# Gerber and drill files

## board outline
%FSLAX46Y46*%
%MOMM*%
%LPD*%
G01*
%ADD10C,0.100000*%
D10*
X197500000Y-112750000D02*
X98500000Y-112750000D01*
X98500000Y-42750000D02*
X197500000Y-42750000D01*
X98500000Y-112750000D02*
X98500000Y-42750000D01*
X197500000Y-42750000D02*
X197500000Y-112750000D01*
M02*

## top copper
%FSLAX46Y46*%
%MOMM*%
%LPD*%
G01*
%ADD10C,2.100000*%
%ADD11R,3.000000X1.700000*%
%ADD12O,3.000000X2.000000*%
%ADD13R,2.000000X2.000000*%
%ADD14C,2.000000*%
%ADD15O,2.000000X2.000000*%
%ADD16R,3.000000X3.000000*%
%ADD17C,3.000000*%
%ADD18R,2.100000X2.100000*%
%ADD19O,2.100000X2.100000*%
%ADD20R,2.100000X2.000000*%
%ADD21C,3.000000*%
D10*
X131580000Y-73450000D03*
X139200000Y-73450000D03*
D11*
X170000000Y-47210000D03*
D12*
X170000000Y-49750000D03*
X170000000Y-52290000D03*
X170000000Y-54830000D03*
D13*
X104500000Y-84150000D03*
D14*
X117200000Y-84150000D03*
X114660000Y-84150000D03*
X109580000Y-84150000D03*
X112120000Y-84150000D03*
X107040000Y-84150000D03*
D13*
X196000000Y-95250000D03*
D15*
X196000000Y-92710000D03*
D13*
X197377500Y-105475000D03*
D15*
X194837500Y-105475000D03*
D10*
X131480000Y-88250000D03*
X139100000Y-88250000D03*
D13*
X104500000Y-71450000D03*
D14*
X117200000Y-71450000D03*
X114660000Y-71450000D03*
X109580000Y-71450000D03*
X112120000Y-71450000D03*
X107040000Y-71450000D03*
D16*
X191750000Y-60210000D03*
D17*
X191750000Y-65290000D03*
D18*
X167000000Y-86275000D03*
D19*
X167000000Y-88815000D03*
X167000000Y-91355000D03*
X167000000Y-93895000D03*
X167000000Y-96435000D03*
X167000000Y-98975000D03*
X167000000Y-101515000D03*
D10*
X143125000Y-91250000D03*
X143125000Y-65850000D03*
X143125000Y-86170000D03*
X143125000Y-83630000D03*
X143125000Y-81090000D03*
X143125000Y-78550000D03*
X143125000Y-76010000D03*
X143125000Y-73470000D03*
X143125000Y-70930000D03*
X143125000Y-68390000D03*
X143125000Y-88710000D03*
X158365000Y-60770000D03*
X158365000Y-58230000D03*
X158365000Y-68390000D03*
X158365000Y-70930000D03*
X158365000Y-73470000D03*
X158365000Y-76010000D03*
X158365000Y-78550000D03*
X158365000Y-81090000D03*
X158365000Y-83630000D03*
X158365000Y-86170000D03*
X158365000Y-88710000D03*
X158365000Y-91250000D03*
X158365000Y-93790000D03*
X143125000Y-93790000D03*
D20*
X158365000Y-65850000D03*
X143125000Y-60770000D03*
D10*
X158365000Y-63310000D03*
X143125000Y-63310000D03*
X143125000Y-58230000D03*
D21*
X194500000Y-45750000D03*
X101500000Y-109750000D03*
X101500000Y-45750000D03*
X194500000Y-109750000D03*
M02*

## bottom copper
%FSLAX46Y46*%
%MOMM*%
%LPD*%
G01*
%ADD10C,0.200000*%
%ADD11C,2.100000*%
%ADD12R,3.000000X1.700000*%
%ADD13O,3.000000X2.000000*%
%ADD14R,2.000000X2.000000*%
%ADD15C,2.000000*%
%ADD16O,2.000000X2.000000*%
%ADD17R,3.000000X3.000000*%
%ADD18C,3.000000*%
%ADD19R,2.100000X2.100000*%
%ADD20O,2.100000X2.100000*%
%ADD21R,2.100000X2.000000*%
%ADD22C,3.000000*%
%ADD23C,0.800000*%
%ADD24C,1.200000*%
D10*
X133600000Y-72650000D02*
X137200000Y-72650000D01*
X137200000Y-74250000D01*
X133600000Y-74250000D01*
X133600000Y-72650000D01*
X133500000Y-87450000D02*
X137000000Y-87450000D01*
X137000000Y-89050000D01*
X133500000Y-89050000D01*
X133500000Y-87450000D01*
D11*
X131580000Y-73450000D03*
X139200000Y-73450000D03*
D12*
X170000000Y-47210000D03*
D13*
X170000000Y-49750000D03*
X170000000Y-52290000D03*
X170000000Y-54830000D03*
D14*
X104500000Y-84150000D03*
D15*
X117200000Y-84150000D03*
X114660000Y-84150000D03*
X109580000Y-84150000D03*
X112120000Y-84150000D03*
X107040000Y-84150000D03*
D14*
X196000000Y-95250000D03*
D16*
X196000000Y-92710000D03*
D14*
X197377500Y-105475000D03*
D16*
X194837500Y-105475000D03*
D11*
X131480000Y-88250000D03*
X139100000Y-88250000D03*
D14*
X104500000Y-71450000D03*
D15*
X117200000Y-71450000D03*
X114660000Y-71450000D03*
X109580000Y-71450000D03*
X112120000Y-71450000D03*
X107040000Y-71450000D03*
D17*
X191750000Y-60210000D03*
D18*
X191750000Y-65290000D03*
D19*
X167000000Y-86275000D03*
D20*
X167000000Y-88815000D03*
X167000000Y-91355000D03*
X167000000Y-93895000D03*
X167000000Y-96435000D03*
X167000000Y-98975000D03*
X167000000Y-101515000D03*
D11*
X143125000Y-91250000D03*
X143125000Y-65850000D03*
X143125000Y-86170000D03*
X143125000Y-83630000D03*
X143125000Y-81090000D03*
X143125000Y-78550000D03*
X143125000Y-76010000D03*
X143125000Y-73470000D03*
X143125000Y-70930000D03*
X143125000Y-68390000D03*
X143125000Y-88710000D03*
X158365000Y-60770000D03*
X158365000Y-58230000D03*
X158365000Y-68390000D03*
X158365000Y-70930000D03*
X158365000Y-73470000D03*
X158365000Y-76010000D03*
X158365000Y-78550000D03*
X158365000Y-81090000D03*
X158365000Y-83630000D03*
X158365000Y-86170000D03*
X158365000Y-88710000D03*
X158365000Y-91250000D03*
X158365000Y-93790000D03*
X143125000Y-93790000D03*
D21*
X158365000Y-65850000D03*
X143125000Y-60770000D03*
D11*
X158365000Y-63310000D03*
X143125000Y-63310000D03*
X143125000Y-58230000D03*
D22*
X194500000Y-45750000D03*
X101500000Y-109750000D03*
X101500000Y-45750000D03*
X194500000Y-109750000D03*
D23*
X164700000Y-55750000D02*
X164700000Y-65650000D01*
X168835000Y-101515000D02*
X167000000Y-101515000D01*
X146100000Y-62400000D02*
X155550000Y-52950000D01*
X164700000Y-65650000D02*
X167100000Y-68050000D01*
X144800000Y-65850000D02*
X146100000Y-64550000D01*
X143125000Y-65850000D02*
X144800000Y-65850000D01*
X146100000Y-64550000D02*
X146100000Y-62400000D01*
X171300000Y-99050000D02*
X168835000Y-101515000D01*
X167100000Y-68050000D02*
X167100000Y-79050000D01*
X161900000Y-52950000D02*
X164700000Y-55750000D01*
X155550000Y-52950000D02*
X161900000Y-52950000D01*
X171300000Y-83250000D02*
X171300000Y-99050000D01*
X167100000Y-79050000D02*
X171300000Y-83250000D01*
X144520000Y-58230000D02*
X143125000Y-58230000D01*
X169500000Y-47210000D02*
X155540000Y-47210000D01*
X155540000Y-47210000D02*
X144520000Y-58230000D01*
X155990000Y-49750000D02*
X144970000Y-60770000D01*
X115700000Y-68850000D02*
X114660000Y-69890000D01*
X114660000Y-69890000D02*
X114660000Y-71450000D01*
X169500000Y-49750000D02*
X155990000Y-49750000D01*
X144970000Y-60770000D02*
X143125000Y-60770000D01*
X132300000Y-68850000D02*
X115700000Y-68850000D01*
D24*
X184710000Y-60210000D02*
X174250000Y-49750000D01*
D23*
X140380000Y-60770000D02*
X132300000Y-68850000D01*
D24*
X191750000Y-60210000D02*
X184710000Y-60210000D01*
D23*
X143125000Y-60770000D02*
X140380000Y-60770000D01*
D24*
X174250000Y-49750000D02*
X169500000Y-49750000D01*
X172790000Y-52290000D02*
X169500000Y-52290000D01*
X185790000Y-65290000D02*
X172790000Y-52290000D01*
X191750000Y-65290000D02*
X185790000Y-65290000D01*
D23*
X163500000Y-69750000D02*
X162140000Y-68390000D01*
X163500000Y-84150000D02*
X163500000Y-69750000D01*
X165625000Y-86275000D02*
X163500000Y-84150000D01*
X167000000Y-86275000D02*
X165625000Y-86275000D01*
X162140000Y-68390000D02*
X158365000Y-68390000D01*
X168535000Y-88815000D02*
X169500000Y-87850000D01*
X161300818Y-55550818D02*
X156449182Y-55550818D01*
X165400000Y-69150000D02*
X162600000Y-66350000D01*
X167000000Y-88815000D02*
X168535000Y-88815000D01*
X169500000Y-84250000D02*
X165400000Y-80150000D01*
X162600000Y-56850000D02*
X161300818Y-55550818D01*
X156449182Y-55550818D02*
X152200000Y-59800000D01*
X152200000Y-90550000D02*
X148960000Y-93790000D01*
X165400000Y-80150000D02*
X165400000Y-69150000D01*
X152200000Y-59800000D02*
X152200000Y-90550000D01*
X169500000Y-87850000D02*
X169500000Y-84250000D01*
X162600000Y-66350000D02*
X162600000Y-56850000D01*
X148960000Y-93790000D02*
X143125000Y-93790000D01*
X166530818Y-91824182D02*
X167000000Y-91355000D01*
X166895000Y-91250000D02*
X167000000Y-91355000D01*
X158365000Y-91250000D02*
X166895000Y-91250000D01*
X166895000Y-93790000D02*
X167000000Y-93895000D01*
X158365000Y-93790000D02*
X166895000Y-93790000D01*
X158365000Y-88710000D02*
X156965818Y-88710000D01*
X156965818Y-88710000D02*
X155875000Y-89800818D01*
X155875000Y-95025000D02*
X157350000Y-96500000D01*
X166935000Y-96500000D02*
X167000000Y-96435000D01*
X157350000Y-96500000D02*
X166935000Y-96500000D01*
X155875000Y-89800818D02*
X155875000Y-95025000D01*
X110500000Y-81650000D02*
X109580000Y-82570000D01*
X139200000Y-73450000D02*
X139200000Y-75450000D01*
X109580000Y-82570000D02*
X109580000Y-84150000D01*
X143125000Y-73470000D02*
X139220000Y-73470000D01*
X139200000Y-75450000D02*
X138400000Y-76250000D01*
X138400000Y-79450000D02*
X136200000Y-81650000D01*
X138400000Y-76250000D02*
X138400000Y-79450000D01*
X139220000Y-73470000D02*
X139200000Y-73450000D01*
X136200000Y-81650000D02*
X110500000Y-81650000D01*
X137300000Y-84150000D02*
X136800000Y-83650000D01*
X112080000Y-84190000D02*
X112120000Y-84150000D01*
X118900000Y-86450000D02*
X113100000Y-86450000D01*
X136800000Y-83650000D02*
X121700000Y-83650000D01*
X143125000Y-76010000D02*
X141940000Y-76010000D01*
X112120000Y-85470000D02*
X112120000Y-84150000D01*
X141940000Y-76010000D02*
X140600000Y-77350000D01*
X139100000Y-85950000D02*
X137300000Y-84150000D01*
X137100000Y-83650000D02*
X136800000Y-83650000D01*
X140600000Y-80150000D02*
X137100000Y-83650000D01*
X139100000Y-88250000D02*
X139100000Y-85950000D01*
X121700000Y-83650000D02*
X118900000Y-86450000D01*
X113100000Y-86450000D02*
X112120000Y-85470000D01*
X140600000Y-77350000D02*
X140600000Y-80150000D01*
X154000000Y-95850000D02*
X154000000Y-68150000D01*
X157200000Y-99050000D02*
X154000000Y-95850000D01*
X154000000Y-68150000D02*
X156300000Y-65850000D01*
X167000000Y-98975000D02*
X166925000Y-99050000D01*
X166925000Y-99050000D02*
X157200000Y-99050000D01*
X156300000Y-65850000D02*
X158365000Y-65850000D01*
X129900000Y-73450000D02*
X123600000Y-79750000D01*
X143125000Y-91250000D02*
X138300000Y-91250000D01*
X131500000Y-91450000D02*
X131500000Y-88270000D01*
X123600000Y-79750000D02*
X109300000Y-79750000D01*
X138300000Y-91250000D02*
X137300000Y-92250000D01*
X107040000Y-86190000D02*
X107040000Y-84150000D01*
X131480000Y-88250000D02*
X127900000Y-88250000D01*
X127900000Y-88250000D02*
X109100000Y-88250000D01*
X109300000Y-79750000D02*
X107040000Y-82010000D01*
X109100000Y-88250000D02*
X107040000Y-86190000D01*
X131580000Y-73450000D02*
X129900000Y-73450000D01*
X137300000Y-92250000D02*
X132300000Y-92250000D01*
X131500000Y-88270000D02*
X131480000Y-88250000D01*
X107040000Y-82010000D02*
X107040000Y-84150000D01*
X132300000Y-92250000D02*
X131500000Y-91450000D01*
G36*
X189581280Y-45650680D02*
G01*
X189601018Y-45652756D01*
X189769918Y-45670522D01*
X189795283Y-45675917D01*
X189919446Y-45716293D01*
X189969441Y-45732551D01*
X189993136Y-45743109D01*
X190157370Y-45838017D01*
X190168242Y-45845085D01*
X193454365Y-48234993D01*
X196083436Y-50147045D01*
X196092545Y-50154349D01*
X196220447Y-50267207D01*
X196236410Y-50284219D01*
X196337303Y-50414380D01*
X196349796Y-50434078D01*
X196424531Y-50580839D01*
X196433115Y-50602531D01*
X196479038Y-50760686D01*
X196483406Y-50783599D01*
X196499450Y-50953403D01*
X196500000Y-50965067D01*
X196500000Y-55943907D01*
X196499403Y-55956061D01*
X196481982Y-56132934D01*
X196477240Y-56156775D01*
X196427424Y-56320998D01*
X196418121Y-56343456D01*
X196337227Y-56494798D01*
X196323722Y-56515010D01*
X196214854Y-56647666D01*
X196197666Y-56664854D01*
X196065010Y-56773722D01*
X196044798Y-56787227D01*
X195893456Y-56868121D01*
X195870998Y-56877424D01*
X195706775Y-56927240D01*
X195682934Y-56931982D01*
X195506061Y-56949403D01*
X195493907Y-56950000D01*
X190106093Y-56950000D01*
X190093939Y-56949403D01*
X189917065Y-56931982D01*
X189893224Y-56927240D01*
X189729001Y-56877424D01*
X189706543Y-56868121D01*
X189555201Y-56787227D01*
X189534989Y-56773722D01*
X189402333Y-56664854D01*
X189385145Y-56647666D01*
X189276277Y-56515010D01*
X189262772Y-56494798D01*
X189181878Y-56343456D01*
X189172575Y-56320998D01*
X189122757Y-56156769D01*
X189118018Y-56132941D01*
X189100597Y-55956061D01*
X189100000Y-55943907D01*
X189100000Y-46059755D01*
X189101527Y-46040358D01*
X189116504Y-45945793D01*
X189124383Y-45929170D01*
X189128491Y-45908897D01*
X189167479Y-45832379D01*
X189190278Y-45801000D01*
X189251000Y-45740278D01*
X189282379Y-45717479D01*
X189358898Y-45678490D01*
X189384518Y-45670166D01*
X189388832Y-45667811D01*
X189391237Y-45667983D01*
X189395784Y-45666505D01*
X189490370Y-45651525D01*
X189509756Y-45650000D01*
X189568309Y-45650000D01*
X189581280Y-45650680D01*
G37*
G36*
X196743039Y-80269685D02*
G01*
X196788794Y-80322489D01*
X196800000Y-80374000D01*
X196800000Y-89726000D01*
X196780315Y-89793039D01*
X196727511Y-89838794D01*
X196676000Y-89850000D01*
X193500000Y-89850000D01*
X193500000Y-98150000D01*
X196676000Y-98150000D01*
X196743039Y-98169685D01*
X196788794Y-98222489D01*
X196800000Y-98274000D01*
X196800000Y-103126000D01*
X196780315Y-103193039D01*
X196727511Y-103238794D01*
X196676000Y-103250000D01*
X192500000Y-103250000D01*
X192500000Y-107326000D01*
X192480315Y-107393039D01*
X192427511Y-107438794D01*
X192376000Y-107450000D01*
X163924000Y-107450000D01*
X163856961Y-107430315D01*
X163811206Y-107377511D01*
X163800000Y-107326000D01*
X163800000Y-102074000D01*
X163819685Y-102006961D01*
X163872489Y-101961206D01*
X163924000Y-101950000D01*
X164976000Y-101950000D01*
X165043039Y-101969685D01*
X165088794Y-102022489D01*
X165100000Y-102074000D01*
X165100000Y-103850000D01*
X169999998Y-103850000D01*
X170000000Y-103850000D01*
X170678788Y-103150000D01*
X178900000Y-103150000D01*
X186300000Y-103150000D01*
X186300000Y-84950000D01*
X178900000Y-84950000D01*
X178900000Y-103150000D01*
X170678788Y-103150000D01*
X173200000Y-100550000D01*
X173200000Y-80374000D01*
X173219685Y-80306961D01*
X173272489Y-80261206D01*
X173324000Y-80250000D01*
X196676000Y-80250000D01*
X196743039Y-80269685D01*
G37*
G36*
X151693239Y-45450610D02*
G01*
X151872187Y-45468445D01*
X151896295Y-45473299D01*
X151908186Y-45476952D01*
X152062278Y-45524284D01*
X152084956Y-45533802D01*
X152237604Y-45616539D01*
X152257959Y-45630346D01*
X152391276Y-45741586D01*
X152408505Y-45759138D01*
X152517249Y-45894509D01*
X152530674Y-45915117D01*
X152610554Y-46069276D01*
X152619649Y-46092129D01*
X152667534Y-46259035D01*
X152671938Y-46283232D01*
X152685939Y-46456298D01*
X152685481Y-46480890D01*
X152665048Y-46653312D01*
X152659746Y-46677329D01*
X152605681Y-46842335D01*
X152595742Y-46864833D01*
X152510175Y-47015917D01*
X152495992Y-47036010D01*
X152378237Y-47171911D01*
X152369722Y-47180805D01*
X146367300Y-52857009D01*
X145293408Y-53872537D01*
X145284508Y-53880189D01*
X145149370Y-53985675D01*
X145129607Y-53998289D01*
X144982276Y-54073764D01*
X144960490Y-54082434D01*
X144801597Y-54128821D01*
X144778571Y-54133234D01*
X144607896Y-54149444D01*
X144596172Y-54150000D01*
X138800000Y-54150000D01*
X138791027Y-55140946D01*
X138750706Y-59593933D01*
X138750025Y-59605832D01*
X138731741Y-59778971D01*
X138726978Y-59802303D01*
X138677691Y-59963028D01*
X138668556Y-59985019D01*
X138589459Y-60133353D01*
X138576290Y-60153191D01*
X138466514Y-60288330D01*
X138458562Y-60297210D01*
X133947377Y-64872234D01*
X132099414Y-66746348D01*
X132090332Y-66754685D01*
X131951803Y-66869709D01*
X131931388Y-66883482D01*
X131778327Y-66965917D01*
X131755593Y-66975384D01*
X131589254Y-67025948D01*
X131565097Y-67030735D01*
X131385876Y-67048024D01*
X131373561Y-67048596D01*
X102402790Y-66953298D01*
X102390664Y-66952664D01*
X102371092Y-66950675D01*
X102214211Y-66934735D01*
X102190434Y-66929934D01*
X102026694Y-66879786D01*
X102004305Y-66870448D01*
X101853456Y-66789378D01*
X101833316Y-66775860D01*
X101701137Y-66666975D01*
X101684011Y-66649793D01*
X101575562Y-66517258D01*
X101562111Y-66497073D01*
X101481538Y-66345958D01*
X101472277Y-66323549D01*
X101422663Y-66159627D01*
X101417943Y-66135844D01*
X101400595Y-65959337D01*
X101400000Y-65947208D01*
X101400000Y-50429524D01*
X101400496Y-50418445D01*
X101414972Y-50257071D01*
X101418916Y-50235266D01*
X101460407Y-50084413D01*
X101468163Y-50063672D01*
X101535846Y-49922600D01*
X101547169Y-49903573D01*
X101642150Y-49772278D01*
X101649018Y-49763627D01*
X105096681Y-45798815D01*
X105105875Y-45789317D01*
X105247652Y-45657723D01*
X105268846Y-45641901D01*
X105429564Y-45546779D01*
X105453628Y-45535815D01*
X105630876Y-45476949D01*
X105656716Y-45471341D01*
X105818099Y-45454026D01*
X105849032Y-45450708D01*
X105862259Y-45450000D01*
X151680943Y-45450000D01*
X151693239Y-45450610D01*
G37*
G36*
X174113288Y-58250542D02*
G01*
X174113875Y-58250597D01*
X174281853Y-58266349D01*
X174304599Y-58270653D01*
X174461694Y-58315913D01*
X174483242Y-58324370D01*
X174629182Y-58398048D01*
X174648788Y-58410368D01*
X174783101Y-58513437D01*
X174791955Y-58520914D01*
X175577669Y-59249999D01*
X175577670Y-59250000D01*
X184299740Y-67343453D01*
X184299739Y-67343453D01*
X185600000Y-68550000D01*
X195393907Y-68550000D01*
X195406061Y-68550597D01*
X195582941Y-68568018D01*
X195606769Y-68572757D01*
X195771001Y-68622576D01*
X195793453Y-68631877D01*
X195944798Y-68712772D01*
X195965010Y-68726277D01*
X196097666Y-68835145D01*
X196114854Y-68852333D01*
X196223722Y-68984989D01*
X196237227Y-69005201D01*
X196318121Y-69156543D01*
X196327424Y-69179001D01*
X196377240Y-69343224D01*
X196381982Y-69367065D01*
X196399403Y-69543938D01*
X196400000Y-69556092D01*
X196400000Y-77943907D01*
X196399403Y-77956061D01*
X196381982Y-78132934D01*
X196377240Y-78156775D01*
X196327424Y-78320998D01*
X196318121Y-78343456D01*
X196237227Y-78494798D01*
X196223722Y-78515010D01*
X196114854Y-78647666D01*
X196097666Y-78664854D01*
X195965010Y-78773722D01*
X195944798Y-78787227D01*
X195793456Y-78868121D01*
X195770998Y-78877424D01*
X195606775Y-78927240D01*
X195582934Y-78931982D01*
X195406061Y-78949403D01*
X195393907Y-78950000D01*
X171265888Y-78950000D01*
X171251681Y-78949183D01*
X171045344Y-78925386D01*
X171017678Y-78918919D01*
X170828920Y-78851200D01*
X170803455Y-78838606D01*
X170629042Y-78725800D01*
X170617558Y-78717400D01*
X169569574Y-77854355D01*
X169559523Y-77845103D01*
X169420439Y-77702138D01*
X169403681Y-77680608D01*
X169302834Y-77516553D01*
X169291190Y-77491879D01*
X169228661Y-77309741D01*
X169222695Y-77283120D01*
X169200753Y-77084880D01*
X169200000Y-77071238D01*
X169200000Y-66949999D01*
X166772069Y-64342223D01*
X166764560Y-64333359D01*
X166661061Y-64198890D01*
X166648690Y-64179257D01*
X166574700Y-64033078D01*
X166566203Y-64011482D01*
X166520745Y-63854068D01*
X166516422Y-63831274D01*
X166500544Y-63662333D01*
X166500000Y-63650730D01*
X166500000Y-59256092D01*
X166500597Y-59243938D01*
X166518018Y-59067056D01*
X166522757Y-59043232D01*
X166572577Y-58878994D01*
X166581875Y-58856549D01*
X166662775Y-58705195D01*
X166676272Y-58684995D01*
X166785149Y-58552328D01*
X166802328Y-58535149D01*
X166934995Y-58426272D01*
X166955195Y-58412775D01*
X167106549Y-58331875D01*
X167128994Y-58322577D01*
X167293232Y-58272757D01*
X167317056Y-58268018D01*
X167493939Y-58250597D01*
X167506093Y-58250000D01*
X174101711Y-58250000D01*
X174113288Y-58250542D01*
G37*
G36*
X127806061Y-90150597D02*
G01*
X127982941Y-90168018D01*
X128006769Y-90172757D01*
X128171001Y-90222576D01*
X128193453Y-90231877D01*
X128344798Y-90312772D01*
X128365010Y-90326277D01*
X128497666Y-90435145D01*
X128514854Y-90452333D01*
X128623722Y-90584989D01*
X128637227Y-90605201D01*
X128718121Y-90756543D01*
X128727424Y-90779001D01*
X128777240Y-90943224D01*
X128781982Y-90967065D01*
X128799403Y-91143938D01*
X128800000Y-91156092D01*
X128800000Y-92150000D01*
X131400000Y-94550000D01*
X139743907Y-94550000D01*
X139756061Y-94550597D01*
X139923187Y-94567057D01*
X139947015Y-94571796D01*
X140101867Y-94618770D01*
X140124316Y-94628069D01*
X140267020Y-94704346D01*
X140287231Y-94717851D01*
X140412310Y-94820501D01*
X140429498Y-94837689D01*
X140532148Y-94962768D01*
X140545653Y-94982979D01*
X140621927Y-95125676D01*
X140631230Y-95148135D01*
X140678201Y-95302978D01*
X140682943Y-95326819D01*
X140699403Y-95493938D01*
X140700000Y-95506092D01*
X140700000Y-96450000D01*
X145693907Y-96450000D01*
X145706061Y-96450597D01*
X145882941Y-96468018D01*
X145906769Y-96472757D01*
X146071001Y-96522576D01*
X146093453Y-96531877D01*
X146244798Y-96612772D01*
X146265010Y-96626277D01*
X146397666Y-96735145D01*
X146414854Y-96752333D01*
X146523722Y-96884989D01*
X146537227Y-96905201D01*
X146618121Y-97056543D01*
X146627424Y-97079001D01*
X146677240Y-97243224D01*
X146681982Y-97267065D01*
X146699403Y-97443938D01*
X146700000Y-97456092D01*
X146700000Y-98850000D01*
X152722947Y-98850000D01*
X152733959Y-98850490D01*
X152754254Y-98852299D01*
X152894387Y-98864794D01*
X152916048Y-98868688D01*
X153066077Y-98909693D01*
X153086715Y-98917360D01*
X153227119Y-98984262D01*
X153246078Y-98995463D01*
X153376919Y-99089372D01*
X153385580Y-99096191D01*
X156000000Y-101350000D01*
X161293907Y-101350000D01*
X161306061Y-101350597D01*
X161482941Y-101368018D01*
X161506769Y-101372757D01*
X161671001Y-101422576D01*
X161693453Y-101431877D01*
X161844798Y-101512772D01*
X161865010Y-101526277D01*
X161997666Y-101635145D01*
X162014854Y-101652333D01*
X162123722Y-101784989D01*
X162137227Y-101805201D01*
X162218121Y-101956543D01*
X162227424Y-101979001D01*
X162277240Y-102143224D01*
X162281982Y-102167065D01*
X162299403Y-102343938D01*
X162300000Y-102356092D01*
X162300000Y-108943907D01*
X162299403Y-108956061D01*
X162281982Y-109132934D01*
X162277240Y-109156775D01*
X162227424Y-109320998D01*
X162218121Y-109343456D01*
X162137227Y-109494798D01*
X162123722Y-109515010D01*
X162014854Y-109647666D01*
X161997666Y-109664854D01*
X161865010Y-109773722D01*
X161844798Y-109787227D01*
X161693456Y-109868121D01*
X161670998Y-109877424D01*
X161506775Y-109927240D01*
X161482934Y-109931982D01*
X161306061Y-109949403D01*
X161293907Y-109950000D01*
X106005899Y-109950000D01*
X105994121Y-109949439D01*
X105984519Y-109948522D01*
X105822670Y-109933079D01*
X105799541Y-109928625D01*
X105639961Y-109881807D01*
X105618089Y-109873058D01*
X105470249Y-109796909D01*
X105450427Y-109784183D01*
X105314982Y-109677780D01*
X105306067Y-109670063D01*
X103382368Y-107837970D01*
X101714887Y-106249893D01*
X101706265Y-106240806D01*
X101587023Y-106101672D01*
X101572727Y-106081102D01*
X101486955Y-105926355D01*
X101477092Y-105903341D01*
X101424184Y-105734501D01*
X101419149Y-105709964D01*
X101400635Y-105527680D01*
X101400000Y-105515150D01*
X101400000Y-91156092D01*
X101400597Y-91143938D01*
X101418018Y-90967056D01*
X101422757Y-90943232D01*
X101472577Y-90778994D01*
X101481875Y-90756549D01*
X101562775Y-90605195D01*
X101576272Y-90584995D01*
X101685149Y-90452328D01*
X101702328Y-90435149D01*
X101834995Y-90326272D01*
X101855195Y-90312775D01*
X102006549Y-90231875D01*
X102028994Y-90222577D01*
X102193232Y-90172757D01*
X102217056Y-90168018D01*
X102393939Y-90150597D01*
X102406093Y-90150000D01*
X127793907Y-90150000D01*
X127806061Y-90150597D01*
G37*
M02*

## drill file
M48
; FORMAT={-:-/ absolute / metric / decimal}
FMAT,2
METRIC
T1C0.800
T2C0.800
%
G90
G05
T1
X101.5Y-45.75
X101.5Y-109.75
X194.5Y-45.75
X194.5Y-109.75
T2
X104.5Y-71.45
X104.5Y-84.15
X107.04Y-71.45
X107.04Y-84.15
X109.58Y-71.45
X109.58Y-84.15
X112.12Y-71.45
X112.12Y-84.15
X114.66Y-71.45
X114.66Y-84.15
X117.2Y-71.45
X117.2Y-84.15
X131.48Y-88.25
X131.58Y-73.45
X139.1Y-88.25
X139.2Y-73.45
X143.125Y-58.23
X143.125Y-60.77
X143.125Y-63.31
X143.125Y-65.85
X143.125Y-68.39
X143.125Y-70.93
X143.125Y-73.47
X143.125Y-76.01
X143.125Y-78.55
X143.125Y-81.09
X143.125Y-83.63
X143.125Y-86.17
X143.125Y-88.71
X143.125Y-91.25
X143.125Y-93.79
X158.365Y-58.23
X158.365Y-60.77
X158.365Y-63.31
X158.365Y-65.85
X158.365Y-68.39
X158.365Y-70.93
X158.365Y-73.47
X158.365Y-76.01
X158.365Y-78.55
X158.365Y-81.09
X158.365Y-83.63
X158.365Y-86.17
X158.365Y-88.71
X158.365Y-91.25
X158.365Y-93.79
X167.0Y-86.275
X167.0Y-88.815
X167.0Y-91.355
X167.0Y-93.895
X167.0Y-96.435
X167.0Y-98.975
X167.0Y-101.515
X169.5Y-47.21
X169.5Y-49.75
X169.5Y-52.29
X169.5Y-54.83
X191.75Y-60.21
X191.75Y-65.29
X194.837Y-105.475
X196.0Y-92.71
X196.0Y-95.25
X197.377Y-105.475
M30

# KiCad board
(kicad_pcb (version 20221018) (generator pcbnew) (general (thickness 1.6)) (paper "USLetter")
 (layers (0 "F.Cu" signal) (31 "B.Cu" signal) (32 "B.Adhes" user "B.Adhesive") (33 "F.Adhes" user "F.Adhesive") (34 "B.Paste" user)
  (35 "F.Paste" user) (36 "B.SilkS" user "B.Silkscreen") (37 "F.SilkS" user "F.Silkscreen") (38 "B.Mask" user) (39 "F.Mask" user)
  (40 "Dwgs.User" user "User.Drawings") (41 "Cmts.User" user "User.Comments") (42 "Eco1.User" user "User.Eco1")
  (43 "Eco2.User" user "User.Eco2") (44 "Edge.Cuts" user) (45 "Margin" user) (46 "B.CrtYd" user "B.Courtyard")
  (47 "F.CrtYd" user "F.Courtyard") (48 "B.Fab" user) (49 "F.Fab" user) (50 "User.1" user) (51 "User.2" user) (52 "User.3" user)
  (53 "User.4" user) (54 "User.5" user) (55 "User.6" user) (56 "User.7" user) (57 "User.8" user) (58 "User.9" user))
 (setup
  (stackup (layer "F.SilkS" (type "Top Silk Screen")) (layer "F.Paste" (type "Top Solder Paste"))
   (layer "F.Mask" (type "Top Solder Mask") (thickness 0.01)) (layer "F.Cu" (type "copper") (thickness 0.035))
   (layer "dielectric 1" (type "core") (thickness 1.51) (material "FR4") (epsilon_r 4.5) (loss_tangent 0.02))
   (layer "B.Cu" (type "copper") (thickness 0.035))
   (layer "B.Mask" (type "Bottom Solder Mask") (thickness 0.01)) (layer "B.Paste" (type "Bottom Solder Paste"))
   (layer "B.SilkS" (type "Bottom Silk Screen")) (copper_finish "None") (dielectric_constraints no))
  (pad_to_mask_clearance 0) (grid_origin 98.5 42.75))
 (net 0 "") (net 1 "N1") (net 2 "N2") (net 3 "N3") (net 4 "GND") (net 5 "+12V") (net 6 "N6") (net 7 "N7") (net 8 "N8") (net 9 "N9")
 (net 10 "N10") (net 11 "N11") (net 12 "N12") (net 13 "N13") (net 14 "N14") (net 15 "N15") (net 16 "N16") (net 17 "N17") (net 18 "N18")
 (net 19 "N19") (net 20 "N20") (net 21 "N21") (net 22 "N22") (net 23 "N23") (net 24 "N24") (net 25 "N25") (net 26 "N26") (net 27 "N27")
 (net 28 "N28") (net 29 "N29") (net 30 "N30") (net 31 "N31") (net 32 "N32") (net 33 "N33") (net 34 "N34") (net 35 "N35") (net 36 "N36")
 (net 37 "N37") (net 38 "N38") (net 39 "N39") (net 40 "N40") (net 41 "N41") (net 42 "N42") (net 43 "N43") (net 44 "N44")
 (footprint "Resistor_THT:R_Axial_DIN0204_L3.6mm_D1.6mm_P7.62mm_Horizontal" (layer "F.Cu") (at 131.58 73.45)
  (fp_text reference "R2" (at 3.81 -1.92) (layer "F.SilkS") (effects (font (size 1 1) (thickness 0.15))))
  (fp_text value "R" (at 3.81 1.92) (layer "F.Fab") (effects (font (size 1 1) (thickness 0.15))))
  (pad "1" thru_hole circle (at 0 0) (size 2.1 2.1) (drill 0.8) (layers "*.Cu" "*.Mask") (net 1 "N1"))
  (pad "2" thru_hole circle (at 7.62 0) (size 2.1 2.1) (drill 0.8) (layers "*.Cu" "*.Mask") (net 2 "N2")))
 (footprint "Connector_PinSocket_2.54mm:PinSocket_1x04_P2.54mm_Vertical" (layer "F.Cu") (at 169.5 47.21)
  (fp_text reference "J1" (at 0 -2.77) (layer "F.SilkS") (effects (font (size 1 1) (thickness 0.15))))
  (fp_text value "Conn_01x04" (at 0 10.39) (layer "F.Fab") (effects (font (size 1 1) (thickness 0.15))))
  (pad "1" thru_hole rect (at 0 0) (size 3 1.7) (drill 0.8 (offset 0.5 0)) (layers "*.Cu" "*.Mask") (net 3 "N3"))
  (pad "2" thru_hole oval (at 0 2.54) (size 3 2) (drill 0.8 (offset 0.5 0)) (layers "*.Cu" "*.Mask") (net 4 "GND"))
  (pad "3" thru_hole oval (at 0 5.08) (size 3 2) (drill 0.8 (offset 0.5 0)) (layers "*.Cu" "*.Mask") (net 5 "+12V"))
  (pad "4" thru_hole oval (at 0 7.62) (size 3 2) (drill 0.8 (offset 0.5 0)) (layers "*.Cu" "*.Mask") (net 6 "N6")))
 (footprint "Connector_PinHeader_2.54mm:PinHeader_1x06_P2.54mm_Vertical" (layer "F.Cu") (at 104.5 84.15 90)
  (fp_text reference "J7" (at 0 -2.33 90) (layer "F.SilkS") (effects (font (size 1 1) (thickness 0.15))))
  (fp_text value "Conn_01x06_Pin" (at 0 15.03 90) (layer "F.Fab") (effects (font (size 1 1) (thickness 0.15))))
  (pad "D2" thru_hole rect (at 0 0 90) (size 2 2) (drill 0.8) (layers "*.Cu" "*.Mask") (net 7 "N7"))
  (pad "D3" thru_hole circle (at 0 12.7 90) (size 2 2) (drill 0.8) (layers "*.Cu" "*.Mask") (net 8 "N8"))
  (pad "GND" thru_hole circle (at 0 10.16 90) (size 2 2) (drill 0.8) (layers "*.Cu" "*.Mask") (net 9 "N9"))
  (pad "SCL" thru_hole circle (at 0 5.08 90) (size 2 2) (drill 0.8) (layers "*.Cu" "*.Mask") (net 2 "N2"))
  (pad "SDA" thru_hole circle (at 0 7.62 90) (size 2 2) (drill 0.8) (layers "*.Cu" "*.Mask") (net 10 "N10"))
  (pad "VCC" thru_hole circle (at 0 2.54 90) (size 2 2) (drill 0.8) (layers "*.Cu" "*.Mask") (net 1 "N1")))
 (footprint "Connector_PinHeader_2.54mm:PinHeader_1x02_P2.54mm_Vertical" (layer "F.Cu") (at 196 95.25 180)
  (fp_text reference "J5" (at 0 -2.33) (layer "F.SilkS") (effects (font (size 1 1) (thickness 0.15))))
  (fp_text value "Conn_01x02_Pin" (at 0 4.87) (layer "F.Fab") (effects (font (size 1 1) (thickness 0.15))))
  (pad "1" thru_hole rect (at 0 0 180) (size 2 2) (drill 0.8) (layers "*.Cu" "*.Mask") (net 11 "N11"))
  (pad "2" thru_hole oval (at 0 2.54 180) (size 2 2) (drill 0.8) (layers "*.Cu" "*.Mask") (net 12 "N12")))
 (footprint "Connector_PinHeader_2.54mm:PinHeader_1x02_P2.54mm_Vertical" (layer "F.Cu") (at 197.3775 105.475 -90)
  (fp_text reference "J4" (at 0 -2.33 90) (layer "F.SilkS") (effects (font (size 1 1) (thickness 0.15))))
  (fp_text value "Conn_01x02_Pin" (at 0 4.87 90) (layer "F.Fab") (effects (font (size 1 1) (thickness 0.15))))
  (pad "1" thru_hole rect (at 0 0 270) (size 2 2) (drill 0.8) (layers "*.Cu" "*.Mask") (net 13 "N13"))
  (pad "2" thru_hole oval (at 0 2.54 270) (size 2 2) (drill 0.8) (layers "*.Cu" "*.Mask") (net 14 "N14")))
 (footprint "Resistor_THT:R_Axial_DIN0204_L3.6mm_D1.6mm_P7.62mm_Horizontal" (layer "F.Cu") (at 131.48 88.25)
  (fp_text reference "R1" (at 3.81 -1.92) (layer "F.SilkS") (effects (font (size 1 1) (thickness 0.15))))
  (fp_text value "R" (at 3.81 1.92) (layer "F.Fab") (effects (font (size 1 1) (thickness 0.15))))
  (pad "1" thru_hole circle (at 0 0) (size 2.1 2.1) (drill 0.8) (layers "*.Cu" "*.Mask") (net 1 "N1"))
  (pad "2" thru_hole circle (at 7.62 0) (size 2.1 2.1) (drill 0.8) (layers "*.Cu" "*.Mask") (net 10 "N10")))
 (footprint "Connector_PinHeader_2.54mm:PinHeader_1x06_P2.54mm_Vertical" (layer "F.Cu") (at 104.5 71.45 90)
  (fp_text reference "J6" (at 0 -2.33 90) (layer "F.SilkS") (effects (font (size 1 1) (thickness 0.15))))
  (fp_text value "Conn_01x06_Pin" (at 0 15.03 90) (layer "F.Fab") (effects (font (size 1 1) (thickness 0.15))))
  (pad "D0" thru_hole rect (at 0 0 90) (size 2 2) (drill 0.8) (layers "*.Cu" "*.Mask") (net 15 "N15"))
  (pad "D1" thru_hole circle (at 0 12.7 90) (size 2 2) (drill 0.8) (layers "*.Cu" "*.Mask") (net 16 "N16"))
  (pad "GND" thru_hole circle (at 0 10.16 90) (size 2 2) (drill 0.8) (layers "*.Cu" "*.Mask") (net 4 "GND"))
  (pad "Rx" thru_hole circle (at 0 5.08 90) (size 2 2) (drill 0.8) (layers "*.Cu" "*.Mask") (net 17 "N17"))
  (pad "Tx" thru_hole circle (at 0 7.62 90) (size 2 2) (drill 0.8) (layers "*.Cu" "*.Mask") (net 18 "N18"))
  (pad "VCC" thru_hole circle (at 0 2.54 90) (size 2 2) (drill 0.8) (layers "*.Cu" "*.Mask") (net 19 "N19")))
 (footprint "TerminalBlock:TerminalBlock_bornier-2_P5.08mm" (layer "F.Cu") (at 191.75 60.21 -90)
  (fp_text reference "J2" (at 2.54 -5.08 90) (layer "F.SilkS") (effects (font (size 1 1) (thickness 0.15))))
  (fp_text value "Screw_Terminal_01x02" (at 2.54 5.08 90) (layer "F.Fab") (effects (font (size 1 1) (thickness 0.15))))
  (pad "1" thru_hole rect (at 0 0 270) (size 3 3) (drill 0.8) (layers "*.Cu" "*.Mask") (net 4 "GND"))
  (pad "2" thru_hole circle (at 5.08 0 270) (size 3 3) (drill 0.8) (layers "*.Cu" "*.Mask") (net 5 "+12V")))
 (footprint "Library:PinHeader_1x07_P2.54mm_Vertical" (layer "F.Cu") (at 167 86.275)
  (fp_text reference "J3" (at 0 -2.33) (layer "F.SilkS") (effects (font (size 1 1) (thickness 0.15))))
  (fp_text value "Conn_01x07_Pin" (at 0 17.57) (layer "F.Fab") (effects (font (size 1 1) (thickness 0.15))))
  (pad "1" thru_hole rect (at 0 0) (size 2.1 2.1) (drill 0.8) (layers "*.Cu" "*.Mask") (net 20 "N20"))
  (pad "2" thru_hole oval (at 0 2.54) (size 2.1 2.1) (drill 0.8) (layers "*.Cu" "*.Mask") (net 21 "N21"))
  (pad "3" thru_hole oval (at 0 5.08) (size 2.1 2.1) (drill 0.8) (layers "*.Cu" "*.Mask") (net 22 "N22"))
  (pad "4" thru_hole oval (at 0 7.62) (size 2.1 2.1) (drill 0.8) (layers "*.Cu" "*.Mask") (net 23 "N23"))
  (pad "5" thru_hole oval (at 0 10.16) (size 2.1 2.1) (drill 0.8) (layers "*.Cu" "*.Mask") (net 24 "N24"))
  (pad "6" thru_hole oval (at 0 12.7) (size 2.1 2.1) (drill 0.8) (layers "*.Cu" "*.Mask") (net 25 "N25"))
  (pad "7" thru_hole oval (at 0 15.24) (size 2.1 2.1) (drill 0.8) (layers "*.Cu" "*.Mask") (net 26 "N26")))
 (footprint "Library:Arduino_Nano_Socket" (layer "B.Cu") (at 150.745 97.6 180)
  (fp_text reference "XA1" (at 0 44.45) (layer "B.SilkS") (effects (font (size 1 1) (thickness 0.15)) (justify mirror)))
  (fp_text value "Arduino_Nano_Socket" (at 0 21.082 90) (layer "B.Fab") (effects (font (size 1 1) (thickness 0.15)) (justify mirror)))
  (pad "3V3" thru_hole circle (at 7.62 6.35 180) (size 2.1 2.1) (drill 0.8) (layers "*.Cu" "*.Mask") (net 1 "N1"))
  (pad "5V" thru_hole circle (at 7.62 31.75 180) (size 2.1 2.1) (drill 0.8) (layers "*.Cu" "*.Mask") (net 26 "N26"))
  (pad "A0" thru_hole circle (at 7.62 11.43 180) (size 2.1 2.1) (drill 0.8) (layers "*.Cu" "*.Mask") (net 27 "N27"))
  (pad "A1" thru_hole circle (at 7.62 13.97 180) (size 2.1 2.1) (drill 0.8) (layers "*.Cu" "*.Mask") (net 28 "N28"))
  (pad "A2" thru_hole circle (at 7.62 16.51 180) (size 2.1 2.1) (drill 0.8) (layers "*.Cu" "*.Mask") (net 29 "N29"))
  (pad "A3" thru_hole circle (at 7.62 19.05 180) (size 2.1 2.1) (drill 0.8) (layers "*.Cu" "*.Mask") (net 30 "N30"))
  (pad "A4" thru_hole circle (at 7.62 21.59 180) (size 2.1 2.1) (drill 0.8) (layers "*.Cu" "*.Mask") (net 10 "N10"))
  (pad "A5" thru_hole circle (at 7.62 24.13 180) (size 2.1 2.1) (drill 0.8) (layers "*.Cu" "*.Mask") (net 2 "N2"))
  (pad "A6" thru_hole circle (at 7.62 26.67 180) (size 2.1 2.1) (drill 0.8) (layers "*.Cu" "*.Mask") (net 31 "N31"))
  (pad "A7" thru_hole circle (at 7.62 29.21 180) (size 2.1 2.1) (drill 0.8) (layers "*.Cu" "*.Mask") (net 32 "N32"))
  (pad "AREF" thru_hole circle (at 7.62 8.89 180) (size 2.1 2.1) (drill 0.8) (layers "*.Cu" "*.Mask") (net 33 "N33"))
  (pad "D0" thru_hole circle (at -7.62 36.83 180) (size 2.1 2.1) (drill 0.8) (layers "*.Cu" "*.Mask") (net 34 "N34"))
  (pad "D1" thru_hole circle (at -7.62 39.37 180) (size 2.1 2.1) (drill 0.8) (layers "*.Cu" "*.Mask") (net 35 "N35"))
  (pad "D2" thru_hole circle (at -7.62 29.21 180) (size 2.1 2.1) (drill 0.8) (layers "*.Cu" "*.Mask") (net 20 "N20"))
  (pad "D3" thru_hole circle (at -7.62 26.67 180) (size 2.1 2.1) (drill 0.8) (layers "*.Cu" "*.Mask") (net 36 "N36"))
  (pad "D4" thru_hole circle (at -7.62 24.13 180) (size 2.1 2.1) (drill 0.8) (layers "*.Cu" "*.Mask") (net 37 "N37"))
  (pad "D5" thru_hole circle (at -7.62 21.59 180) (size 2.1 2.1) (drill 0.8) (layers "*.Cu" "*.Mask") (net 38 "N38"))
  (pad "D6" thru_hole circle (at -7.62 19.05 180) (size 2.1 2.1) (drill 0.8) (layers "*.Cu" "*.Mask") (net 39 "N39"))
  (pad "D7" thru_hole circle (at -7.62 16.51 180) (size 2.1 2.1) (drill 0.8) (layers "*.Cu" "*.Mask") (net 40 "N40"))
  (pad "D8" thru_hole circle (at -7.62 13.97 180) (size 2.1 2.1) (drill 0.8) (layers "*.Cu" "*.Mask") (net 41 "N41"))
  (pad "D9" thru_hole circle (at -7.62 11.43 180) (size 2.1 2.1) (drill 0.8) (layers "*.Cu" "*.Mask") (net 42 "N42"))
  (pad "D10" thru_hole circle (at -7.62 8.89 180) (size 2.1 2.1) (drill 0.8) (layers "*.Cu" "*.Mask") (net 24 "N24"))
  (pad "D11" thru_hole circle (at -7.62 6.35 180) (size 2.1 2.1) (drill 0.8) (layers "*.Cu" "*.Mask") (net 22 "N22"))
  (pad "D12" thru_hole circle (at -7.62 3.81 180) (size 2.1 2.1) (drill 0.8) (layers "*.Cu" "*.Mask") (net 23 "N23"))
  (pad "D13" thru_hole circle (at 7.62 3.81 180) (size 2.1 2.1) (drill 0.8) (layers "*.Cu" "*.Mask") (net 21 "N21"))
  (pad "GND1" thru_hole rect (at -7.62 31.75 180) (size 2.1 2) (drill 0.8) (layers "*.Cu" "*.Mask") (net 25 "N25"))
  (pad "GND2" thru_hole rect (at 7.62 36.83 180) (size 2.1 2) (drill 0.8) (layers "*.Cu" "*.Mask") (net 4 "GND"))
  (pad "RST1" thru_hole circle (at -7.62 34.29 180) (size 2.1 2.1) (drill 0.8) (layers "*.Cu" "*.Mask") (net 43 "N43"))
  (pad "RST2" thru_hole circle (at 7.62 34.29 180) (size 2.1 2.1) (drill 0.8) (layers "*.Cu" "*.Mask") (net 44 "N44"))
  (pad "VIN" thru_hole circle (at 7.62 39.37 180) (size 2.1 2.1) (drill 0.8) (layers "*.Cu" "*.Mask") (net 3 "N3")))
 (gr_rect (start 133.6 72.65) (end 137.2 74.25) (stroke (width 0.2) (type default)) (fill none) (layer "B.Cu"))
 (gr_rect (start 133.5 87.45) (end 137 89.05) (stroke (width 0.2) (type default)) (fill none) (layer "B.Cu"))
 (gr_line (start 197.5 112.75) (end 98.5 112.75) (stroke (width 0.1) (type default)) (layer "Edge.Cuts"))
 (gr_line (start 98.5 42.75) (end 197.5 42.75) (stroke (width 0.1) (type default)) (layer "Edge.Cuts"))
 (gr_line (start 98.5 112.75) (end 98.5 42.75) (stroke (width 0.1) (type default)) (layer "Edge.Cuts"))
 (gr_line (start 197.5 42.75) (end 197.5 112.75) (stroke (width 0.1) (type default)) (layer "Edge.Cuts"))
 (via (at 194.5 45.75) (size 3) (drill 0.8) (layers "F.Cu" "B.Cu") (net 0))
 (via (at 101.5 109.75) (size 3) (drill 0.8) (layers "F.Cu" "B.Cu") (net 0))
 (via (at 101.5 45.75) (size 3) (drill 0.8) (layers "F.Cu" "B.Cu") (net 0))
 (via (at 194.5 109.75) (size 3) (drill 0.8) (layers "F.Cu" "B.Cu") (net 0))
 (segment (start 164.7 55.75) (end 164.7 65.65) (width 0.8) (layer "B.Cu") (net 26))
 (segment (start 168.835 101.515) (end 167 101.515) (width 0.8) (layer "B.Cu") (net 26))
 (segment (start 146.1 62.4) (end 155.55 52.95) (width 0.8) (layer "B.Cu") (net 26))
 (segment (start 164.7 65.65) (end 167.1 68.05) (width 0.8) (layer "B.Cu") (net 26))
 (segment (start 144.8 65.85) (end 146.1 64.55) (width 0.8) (layer "B.Cu") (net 26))
 (segment (start 143.125 65.85) (end 144.8 65.85) (width 0.8) (layer "B.Cu") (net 26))
 (segment (start 146.1 64.55) (end 146.1 62.4) (width 0.8) (layer "B.Cu") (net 26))
 (segment (start 171.3 99.05) (end 168.835 101.515) (width 0.8) (layer "B.Cu") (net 26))
 (segment (start 167.1 68.05) (end 167.1 79.05) (width 0.8) (layer "B.Cu") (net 26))
 (segment (start 161.9 52.95) (end 164.7 55.75) (width 0.8) (layer "B.Cu") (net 26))
 (segment (start 155.55 52.95) (end 161.9 52.95) (width 0.8) (layer "B.Cu") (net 26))
 (segment (start 171.3 83.25) (end 171.3 99.05) (width 0.8) (layer "B.Cu") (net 26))
 (segment (start 167.1 79.05) (end 171.3 83.25) (width 0.8) (layer "B.Cu") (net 26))
 (segment (start 144.52 58.23) (end 143.125 58.23) (width 0.8) (layer "B.Cu") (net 3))
 (segment (start 169.5 47.21) (end 155.54 47.21) (width 0.8) (layer "B.Cu") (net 3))
 (segment (start 155.54 47.21) (end 144.52 58.23) (width 0.8) (layer "B.Cu") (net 3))
 (segment (start 155.99 49.75) (end 144.97 60.77) (width 0.8) (layer "B.Cu") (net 4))
 (segment (start 115.7 68.85) (end 114.66 69.89) (width 0.8) (layer "B.Cu") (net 4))
 (segment (start 114.66 69.89) (end 114.66 71.45) (width 0.8) (layer "B.Cu") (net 4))
 (segment (start 169.5 49.75) (end 155.99 49.75) (width 0.8) (layer "B.Cu") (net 4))
 (segment (start 144.97 60.77) (end 143.125 60.77) (width 0.8) (layer "B.Cu") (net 4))
 (segment (start 132.3 68.85) (end 115.7 68.85) (width 0.8) (layer "B.Cu") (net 4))
 (segment (start 184.71 60.21) (end 174.25 49.75) (width 1.2) (layer "B.Cu") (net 4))
 (segment (start 140.38 60.77) (end 132.3 68.85) (width 0.8) (layer "B.Cu") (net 4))
 (segment (start 191.75 60.21) (end 184.71 60.21) (width 1.2) (layer "B.Cu") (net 4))
 (segment (start 143.125 60.77) (end 140.38 60.77) (width 0.8) (layer "B.Cu") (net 4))
 (segment (start 174.25 49.75) (end 169.5 49.75) (width 1.2) (layer "B.Cu") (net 4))
 (segment (start 172.79 52.29) (end 169.5 52.29) (width 1.2) (layer "B.Cu") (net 5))
 (segment (start 185.79 65.29) (end 172.79 52.29) (width 1.2) (layer "B.Cu") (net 5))
 (segment (start 191.75 65.29) (end 185.79 65.29) (width 1.2) (layer "B.Cu") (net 5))
 (segment (start 163.5 69.75) (end 162.14 68.39) (width 0.8) (layer "B.Cu") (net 20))
 (segment (start 163.5 84.15) (end 163.5 69.75) (width 0.8) (layer "B.Cu") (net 20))
 (segment (start 165.625 86.275) (end 163.5 84.15) (width 0.8) (layer "B.Cu") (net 20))
 (segment (start 167 86.275) (end 165.625 86.275) (width 0.8) (layer "B.Cu") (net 20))
 (segment (start 162.14 68.39) (end 158.365 68.39) (width 0.8) (layer "B.Cu") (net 20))
 (segment (start 168.535 88.815) (end 169.5 87.85) (width 0.8) (layer "B.Cu") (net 21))
 (segment (start 161.300818 55.550818) (end 156.449182 55.550818) (width 0.8) (layer "B.Cu") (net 21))
 (segment (start 165.4 69.15) (end 162.6 66.35) (width 0.8) (layer "B.Cu") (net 21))
 (segment (start 167 88.815) (end 168.535 88.815) (width 0.8) (layer "B.Cu") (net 21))
 (segment (start 169.5 84.25) (end 165.4 80.15) (width 0.8) (layer "B.Cu") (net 21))
 (segment (start 162.6 56.85) (end 161.300818 55.550818) (width 0.8) (layer "B.Cu") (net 21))
 (segment (start 156.449182 55.550818) (end 152.2 59.8) (width 0.8) (layer "B.Cu") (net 21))
 (segment (start 152.2 90.55) (end 148.96 93.79) (width 0.8) (layer "B.Cu") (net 21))
 (segment (start 165.4 80.15) (end 165.4 69.15) (width 0.8) (layer "B.Cu") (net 21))
 (segment (start 152.2 59.8) (end 152.2 90.55) (width 0.8) (layer "B.Cu") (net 21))
 (segment (start 169.5 87.85) (end 169.5 84.25) (width 0.8) (layer "B.Cu") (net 21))
 (segment (start 162.6 66.35) (end 162.6 56.85) (width 0.8) (layer "B.Cu") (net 21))
 (segment (start 148.96 93.79) (end 143.125 93.79) (width 0.8) (layer "B.Cu") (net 21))
 (segment (start 166.530818 91.824182) (end 167 91.355) (width 0.8) (layer "B.Cu") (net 22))
 (segment (start 166.895 91.25) (end 167 91.355) (width 0.8) (layer "B.Cu") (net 22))
 (segment (start 158.365 91.25) (end 166.895 91.25) (width 0.8) (layer "B.Cu") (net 22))
 (segment (start 166.895 93.79) (end 167 93.895) (width 0.8) (layer "B.Cu") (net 23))
 (segment (start 158.365 93.79) (end 166.895 93.79) (width 0.8) (layer "B.Cu") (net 23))
 (segment (start 158.365 88.71) (end 156.965818 88.71) (width 0.8) (layer "B.Cu") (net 24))
 (segment (start 156.965818 88.71) (end 155.875 89.800818) (width 0.8) (layer "B.Cu") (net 24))
 (segment (start 155.875 95.025) (end 157.35 96.5) (width 0.8) (layer "B.Cu") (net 24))
 (segment (start 166.935 96.5) (end 167 96.435) (width 0.8) (layer "B.Cu") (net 24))
 (segment (start 157.35 96.5) (end 166.935 96.5) (width 0.8) (layer "B.Cu") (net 24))
 (segment (start 155.875 89.800818) (end 155.875 95.025) (width 0.8) (layer "B.Cu") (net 24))
 (segment (start 110.5 81.65) (end 109.58 82.57) (width 0.8) (layer "B.Cu") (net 2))
 (segment (start 139.2 73.45) (end 139.2 75.45) (width 0.8) (layer "B.Cu") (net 2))
 (segment (start 109.58 82.57) (end 109.58 84.15) (width 0.8) (layer "B.Cu") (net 2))
 (segment (start 143.125 73.47) (end 139.22 73.47) (width 0.8) (layer "B.Cu") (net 2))
 (segment (start 139.2 75.45) (end 138.4 76.25) (width 0.8) (layer "B.Cu") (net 2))
 (segment (start 138.4 79.45) (end 136.2 81.65) (width 0.8) (layer "B.Cu") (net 2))
 (segment (start 138.4 76.25) (end 138.4 79.45) (width 0.8) (layer "B.Cu") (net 2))
 (segment (start 139.22 73.47) (end 139.2 73.45) (width 0.8) (layer "B.Cu") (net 2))
 (segment (start 136.2 81.65) (end 110.5 81.65) (width 0.8) (layer "B.Cu") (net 2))
 (segment (start 137.3 84.15) (end 136.8 83.65) (width 0.8) (layer "B.Cu") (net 10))
 (segment (start 112.08 84.19) (end 112.12 84.15) (width 0.8) (layer "B.Cu") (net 10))
 (segment (start 118.9 86.45) (end 113.1 86.45) (width 0.8) (layer "B.Cu") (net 10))
 (segment (start 136.8 83.65) (end 121.7 83.65) (width 0.8) (layer "B.Cu") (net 10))
 (segment (start 143.125 76.01) (end 141.94 76.01) (width 0.8) (layer "B.Cu") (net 10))
 (segment (start 112.12 85.47) (end 112.12 84.15) (width 0.8) (layer "B.Cu") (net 10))
 (segment (start 141.94 76.01) (end 140.6 77.35) (width 0.8) (layer "B.Cu") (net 10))
 (segment (start 139.1 85.95) (end 137.3 84.15) (width 0.8) (layer "B.Cu") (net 10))
 (segment (start 137.1 83.65) (end 136.8 83.65) (width 0.8) (layer "B.Cu") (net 10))
 (segment (start 140.6 80.15) (end 137.1 83.65) (width 0.8) (layer "B.Cu") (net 10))
 (segment (start 139.1 88.25) (end 139.1 85.95) (width 0.8) (layer "B.Cu") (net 10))
 (segment (start 121.7 83.65) (end 118.9 86.45) (width 0.8) (layer "B.Cu") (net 10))
 (segment (start 113.1 86.45) (end 112.12 85.47) (width 0.8) (layer "B.Cu") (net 10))
 (segment (start 140.6 77.35) (end 140.6 80.15) (width 0.8) (layer "B.Cu") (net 10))
 (segment (start 154 95.85) (end 154 68.15) (width 0.8) (layer "B.Cu") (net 25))
 (segment (start 157.2 99.05) (end 154 95.85) (width 0.8) (layer "B.Cu") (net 25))
 (segment (start 154 68.15) (end 156.3 65.85) (width 0.8) (layer "B.Cu") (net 25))
 (segment (start 167 98.975) (end 166.925 99.05) (width 0.8) (layer "B.Cu") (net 25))
 (segment (start 166.925 99.05) (end 157.2 99.05) (width 0.8) (layer "B.Cu") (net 25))
 (segment (start 156.3 65.85) (end 158.365 65.85) (width 0.8) (layer "B.Cu") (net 25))
 (segment (start 129.9 73.45) (end 123.6 79.75) (width 0.8) (layer "B.Cu") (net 1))
 (segment (start 143.125 91.25) (end 138.3 91.25) (width 0.8) (layer "B.Cu") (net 1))
 (segment (start 131.5 91.45) (end 131.5 88.27) (width 0.8) (layer "B.Cu") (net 1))
 (segment (start 123.6 79.75) (end 109.3 79.75) (width 0.8) (layer "B.Cu") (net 1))
 (segment (start 138.3 91.25) (end 137.3 92.25) (width 0.8) (layer "B.Cu") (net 1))
 (segment (start 107.04 86.19) (end 107.04 84.15) (width 0.8) (layer "B.Cu") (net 1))
 (segment (start 131.48 88.25) (end 127.9 88.25) (width 0.8) (layer "B.Cu") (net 1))
 (segment (start 127.9 88.25) (end 109.1 88.25) (width 0.8) (layer "B.Cu") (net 1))
 (segment (start 109.3 79.75) (end 107.04 82.01) (width 0.8) (layer "B.Cu") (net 1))
 (segment (start 109.1 88.25) (end 107.04 86.19) (width 0.8) (layer "B.Cu") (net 1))
 (segment (start 131.58 73.45) (end 129.9 73.45) (width 0.8) (layer "B.Cu") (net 1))
 (segment (start 137.3 92.25) (end 132.3 92.25) (width 0.8) (layer "B.Cu") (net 1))
 (segment (start 131.5 88.27) (end 131.48 88.25) (width 0.8) (layer "B.Cu") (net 1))
 (segment (start 107.04 82.01) (end 107.04 84.15) (width 0.8) (layer "B.Cu") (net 1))
 (segment (start 132.3 92.25) (end 131.5 91.45) (width 0.8) (layer "B.Cu") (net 1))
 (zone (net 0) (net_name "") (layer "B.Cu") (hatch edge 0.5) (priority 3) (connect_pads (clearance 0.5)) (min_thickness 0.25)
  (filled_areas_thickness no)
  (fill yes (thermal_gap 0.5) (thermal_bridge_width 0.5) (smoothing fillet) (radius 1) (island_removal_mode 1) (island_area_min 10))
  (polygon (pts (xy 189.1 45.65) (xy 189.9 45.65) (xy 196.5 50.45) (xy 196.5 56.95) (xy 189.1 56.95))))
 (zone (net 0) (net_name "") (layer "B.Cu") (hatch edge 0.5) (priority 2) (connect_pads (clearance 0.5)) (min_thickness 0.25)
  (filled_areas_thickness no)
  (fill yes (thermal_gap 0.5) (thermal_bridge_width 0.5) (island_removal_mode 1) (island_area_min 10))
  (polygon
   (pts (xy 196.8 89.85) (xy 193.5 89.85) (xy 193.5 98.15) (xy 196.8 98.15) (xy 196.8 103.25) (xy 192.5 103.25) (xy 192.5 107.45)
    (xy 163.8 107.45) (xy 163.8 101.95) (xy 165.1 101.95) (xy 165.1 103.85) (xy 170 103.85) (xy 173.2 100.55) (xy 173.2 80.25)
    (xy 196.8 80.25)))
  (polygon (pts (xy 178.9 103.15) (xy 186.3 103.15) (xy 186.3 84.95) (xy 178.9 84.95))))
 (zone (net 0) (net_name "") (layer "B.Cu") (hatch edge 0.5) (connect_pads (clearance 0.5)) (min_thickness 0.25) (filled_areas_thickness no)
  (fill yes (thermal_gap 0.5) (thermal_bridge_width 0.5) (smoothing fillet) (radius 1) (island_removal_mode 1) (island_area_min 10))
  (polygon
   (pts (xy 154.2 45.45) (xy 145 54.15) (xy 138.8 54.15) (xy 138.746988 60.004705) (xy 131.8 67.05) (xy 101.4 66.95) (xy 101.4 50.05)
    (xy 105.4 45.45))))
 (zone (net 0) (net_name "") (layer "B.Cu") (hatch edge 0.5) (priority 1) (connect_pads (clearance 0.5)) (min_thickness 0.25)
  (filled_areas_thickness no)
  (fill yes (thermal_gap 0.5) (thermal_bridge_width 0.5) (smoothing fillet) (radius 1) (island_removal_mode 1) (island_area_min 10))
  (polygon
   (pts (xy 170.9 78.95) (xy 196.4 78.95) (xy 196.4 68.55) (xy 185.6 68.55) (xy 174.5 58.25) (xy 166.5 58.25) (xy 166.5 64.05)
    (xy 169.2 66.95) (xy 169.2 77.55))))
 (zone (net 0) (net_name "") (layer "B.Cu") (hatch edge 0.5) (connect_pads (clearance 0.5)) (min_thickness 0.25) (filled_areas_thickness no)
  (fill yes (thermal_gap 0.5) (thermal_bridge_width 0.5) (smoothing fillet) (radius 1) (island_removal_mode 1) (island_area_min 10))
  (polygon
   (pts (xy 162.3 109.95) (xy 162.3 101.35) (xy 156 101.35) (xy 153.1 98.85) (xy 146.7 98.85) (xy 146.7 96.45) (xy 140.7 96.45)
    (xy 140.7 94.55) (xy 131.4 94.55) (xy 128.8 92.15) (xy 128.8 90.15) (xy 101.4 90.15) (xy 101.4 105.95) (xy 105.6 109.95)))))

